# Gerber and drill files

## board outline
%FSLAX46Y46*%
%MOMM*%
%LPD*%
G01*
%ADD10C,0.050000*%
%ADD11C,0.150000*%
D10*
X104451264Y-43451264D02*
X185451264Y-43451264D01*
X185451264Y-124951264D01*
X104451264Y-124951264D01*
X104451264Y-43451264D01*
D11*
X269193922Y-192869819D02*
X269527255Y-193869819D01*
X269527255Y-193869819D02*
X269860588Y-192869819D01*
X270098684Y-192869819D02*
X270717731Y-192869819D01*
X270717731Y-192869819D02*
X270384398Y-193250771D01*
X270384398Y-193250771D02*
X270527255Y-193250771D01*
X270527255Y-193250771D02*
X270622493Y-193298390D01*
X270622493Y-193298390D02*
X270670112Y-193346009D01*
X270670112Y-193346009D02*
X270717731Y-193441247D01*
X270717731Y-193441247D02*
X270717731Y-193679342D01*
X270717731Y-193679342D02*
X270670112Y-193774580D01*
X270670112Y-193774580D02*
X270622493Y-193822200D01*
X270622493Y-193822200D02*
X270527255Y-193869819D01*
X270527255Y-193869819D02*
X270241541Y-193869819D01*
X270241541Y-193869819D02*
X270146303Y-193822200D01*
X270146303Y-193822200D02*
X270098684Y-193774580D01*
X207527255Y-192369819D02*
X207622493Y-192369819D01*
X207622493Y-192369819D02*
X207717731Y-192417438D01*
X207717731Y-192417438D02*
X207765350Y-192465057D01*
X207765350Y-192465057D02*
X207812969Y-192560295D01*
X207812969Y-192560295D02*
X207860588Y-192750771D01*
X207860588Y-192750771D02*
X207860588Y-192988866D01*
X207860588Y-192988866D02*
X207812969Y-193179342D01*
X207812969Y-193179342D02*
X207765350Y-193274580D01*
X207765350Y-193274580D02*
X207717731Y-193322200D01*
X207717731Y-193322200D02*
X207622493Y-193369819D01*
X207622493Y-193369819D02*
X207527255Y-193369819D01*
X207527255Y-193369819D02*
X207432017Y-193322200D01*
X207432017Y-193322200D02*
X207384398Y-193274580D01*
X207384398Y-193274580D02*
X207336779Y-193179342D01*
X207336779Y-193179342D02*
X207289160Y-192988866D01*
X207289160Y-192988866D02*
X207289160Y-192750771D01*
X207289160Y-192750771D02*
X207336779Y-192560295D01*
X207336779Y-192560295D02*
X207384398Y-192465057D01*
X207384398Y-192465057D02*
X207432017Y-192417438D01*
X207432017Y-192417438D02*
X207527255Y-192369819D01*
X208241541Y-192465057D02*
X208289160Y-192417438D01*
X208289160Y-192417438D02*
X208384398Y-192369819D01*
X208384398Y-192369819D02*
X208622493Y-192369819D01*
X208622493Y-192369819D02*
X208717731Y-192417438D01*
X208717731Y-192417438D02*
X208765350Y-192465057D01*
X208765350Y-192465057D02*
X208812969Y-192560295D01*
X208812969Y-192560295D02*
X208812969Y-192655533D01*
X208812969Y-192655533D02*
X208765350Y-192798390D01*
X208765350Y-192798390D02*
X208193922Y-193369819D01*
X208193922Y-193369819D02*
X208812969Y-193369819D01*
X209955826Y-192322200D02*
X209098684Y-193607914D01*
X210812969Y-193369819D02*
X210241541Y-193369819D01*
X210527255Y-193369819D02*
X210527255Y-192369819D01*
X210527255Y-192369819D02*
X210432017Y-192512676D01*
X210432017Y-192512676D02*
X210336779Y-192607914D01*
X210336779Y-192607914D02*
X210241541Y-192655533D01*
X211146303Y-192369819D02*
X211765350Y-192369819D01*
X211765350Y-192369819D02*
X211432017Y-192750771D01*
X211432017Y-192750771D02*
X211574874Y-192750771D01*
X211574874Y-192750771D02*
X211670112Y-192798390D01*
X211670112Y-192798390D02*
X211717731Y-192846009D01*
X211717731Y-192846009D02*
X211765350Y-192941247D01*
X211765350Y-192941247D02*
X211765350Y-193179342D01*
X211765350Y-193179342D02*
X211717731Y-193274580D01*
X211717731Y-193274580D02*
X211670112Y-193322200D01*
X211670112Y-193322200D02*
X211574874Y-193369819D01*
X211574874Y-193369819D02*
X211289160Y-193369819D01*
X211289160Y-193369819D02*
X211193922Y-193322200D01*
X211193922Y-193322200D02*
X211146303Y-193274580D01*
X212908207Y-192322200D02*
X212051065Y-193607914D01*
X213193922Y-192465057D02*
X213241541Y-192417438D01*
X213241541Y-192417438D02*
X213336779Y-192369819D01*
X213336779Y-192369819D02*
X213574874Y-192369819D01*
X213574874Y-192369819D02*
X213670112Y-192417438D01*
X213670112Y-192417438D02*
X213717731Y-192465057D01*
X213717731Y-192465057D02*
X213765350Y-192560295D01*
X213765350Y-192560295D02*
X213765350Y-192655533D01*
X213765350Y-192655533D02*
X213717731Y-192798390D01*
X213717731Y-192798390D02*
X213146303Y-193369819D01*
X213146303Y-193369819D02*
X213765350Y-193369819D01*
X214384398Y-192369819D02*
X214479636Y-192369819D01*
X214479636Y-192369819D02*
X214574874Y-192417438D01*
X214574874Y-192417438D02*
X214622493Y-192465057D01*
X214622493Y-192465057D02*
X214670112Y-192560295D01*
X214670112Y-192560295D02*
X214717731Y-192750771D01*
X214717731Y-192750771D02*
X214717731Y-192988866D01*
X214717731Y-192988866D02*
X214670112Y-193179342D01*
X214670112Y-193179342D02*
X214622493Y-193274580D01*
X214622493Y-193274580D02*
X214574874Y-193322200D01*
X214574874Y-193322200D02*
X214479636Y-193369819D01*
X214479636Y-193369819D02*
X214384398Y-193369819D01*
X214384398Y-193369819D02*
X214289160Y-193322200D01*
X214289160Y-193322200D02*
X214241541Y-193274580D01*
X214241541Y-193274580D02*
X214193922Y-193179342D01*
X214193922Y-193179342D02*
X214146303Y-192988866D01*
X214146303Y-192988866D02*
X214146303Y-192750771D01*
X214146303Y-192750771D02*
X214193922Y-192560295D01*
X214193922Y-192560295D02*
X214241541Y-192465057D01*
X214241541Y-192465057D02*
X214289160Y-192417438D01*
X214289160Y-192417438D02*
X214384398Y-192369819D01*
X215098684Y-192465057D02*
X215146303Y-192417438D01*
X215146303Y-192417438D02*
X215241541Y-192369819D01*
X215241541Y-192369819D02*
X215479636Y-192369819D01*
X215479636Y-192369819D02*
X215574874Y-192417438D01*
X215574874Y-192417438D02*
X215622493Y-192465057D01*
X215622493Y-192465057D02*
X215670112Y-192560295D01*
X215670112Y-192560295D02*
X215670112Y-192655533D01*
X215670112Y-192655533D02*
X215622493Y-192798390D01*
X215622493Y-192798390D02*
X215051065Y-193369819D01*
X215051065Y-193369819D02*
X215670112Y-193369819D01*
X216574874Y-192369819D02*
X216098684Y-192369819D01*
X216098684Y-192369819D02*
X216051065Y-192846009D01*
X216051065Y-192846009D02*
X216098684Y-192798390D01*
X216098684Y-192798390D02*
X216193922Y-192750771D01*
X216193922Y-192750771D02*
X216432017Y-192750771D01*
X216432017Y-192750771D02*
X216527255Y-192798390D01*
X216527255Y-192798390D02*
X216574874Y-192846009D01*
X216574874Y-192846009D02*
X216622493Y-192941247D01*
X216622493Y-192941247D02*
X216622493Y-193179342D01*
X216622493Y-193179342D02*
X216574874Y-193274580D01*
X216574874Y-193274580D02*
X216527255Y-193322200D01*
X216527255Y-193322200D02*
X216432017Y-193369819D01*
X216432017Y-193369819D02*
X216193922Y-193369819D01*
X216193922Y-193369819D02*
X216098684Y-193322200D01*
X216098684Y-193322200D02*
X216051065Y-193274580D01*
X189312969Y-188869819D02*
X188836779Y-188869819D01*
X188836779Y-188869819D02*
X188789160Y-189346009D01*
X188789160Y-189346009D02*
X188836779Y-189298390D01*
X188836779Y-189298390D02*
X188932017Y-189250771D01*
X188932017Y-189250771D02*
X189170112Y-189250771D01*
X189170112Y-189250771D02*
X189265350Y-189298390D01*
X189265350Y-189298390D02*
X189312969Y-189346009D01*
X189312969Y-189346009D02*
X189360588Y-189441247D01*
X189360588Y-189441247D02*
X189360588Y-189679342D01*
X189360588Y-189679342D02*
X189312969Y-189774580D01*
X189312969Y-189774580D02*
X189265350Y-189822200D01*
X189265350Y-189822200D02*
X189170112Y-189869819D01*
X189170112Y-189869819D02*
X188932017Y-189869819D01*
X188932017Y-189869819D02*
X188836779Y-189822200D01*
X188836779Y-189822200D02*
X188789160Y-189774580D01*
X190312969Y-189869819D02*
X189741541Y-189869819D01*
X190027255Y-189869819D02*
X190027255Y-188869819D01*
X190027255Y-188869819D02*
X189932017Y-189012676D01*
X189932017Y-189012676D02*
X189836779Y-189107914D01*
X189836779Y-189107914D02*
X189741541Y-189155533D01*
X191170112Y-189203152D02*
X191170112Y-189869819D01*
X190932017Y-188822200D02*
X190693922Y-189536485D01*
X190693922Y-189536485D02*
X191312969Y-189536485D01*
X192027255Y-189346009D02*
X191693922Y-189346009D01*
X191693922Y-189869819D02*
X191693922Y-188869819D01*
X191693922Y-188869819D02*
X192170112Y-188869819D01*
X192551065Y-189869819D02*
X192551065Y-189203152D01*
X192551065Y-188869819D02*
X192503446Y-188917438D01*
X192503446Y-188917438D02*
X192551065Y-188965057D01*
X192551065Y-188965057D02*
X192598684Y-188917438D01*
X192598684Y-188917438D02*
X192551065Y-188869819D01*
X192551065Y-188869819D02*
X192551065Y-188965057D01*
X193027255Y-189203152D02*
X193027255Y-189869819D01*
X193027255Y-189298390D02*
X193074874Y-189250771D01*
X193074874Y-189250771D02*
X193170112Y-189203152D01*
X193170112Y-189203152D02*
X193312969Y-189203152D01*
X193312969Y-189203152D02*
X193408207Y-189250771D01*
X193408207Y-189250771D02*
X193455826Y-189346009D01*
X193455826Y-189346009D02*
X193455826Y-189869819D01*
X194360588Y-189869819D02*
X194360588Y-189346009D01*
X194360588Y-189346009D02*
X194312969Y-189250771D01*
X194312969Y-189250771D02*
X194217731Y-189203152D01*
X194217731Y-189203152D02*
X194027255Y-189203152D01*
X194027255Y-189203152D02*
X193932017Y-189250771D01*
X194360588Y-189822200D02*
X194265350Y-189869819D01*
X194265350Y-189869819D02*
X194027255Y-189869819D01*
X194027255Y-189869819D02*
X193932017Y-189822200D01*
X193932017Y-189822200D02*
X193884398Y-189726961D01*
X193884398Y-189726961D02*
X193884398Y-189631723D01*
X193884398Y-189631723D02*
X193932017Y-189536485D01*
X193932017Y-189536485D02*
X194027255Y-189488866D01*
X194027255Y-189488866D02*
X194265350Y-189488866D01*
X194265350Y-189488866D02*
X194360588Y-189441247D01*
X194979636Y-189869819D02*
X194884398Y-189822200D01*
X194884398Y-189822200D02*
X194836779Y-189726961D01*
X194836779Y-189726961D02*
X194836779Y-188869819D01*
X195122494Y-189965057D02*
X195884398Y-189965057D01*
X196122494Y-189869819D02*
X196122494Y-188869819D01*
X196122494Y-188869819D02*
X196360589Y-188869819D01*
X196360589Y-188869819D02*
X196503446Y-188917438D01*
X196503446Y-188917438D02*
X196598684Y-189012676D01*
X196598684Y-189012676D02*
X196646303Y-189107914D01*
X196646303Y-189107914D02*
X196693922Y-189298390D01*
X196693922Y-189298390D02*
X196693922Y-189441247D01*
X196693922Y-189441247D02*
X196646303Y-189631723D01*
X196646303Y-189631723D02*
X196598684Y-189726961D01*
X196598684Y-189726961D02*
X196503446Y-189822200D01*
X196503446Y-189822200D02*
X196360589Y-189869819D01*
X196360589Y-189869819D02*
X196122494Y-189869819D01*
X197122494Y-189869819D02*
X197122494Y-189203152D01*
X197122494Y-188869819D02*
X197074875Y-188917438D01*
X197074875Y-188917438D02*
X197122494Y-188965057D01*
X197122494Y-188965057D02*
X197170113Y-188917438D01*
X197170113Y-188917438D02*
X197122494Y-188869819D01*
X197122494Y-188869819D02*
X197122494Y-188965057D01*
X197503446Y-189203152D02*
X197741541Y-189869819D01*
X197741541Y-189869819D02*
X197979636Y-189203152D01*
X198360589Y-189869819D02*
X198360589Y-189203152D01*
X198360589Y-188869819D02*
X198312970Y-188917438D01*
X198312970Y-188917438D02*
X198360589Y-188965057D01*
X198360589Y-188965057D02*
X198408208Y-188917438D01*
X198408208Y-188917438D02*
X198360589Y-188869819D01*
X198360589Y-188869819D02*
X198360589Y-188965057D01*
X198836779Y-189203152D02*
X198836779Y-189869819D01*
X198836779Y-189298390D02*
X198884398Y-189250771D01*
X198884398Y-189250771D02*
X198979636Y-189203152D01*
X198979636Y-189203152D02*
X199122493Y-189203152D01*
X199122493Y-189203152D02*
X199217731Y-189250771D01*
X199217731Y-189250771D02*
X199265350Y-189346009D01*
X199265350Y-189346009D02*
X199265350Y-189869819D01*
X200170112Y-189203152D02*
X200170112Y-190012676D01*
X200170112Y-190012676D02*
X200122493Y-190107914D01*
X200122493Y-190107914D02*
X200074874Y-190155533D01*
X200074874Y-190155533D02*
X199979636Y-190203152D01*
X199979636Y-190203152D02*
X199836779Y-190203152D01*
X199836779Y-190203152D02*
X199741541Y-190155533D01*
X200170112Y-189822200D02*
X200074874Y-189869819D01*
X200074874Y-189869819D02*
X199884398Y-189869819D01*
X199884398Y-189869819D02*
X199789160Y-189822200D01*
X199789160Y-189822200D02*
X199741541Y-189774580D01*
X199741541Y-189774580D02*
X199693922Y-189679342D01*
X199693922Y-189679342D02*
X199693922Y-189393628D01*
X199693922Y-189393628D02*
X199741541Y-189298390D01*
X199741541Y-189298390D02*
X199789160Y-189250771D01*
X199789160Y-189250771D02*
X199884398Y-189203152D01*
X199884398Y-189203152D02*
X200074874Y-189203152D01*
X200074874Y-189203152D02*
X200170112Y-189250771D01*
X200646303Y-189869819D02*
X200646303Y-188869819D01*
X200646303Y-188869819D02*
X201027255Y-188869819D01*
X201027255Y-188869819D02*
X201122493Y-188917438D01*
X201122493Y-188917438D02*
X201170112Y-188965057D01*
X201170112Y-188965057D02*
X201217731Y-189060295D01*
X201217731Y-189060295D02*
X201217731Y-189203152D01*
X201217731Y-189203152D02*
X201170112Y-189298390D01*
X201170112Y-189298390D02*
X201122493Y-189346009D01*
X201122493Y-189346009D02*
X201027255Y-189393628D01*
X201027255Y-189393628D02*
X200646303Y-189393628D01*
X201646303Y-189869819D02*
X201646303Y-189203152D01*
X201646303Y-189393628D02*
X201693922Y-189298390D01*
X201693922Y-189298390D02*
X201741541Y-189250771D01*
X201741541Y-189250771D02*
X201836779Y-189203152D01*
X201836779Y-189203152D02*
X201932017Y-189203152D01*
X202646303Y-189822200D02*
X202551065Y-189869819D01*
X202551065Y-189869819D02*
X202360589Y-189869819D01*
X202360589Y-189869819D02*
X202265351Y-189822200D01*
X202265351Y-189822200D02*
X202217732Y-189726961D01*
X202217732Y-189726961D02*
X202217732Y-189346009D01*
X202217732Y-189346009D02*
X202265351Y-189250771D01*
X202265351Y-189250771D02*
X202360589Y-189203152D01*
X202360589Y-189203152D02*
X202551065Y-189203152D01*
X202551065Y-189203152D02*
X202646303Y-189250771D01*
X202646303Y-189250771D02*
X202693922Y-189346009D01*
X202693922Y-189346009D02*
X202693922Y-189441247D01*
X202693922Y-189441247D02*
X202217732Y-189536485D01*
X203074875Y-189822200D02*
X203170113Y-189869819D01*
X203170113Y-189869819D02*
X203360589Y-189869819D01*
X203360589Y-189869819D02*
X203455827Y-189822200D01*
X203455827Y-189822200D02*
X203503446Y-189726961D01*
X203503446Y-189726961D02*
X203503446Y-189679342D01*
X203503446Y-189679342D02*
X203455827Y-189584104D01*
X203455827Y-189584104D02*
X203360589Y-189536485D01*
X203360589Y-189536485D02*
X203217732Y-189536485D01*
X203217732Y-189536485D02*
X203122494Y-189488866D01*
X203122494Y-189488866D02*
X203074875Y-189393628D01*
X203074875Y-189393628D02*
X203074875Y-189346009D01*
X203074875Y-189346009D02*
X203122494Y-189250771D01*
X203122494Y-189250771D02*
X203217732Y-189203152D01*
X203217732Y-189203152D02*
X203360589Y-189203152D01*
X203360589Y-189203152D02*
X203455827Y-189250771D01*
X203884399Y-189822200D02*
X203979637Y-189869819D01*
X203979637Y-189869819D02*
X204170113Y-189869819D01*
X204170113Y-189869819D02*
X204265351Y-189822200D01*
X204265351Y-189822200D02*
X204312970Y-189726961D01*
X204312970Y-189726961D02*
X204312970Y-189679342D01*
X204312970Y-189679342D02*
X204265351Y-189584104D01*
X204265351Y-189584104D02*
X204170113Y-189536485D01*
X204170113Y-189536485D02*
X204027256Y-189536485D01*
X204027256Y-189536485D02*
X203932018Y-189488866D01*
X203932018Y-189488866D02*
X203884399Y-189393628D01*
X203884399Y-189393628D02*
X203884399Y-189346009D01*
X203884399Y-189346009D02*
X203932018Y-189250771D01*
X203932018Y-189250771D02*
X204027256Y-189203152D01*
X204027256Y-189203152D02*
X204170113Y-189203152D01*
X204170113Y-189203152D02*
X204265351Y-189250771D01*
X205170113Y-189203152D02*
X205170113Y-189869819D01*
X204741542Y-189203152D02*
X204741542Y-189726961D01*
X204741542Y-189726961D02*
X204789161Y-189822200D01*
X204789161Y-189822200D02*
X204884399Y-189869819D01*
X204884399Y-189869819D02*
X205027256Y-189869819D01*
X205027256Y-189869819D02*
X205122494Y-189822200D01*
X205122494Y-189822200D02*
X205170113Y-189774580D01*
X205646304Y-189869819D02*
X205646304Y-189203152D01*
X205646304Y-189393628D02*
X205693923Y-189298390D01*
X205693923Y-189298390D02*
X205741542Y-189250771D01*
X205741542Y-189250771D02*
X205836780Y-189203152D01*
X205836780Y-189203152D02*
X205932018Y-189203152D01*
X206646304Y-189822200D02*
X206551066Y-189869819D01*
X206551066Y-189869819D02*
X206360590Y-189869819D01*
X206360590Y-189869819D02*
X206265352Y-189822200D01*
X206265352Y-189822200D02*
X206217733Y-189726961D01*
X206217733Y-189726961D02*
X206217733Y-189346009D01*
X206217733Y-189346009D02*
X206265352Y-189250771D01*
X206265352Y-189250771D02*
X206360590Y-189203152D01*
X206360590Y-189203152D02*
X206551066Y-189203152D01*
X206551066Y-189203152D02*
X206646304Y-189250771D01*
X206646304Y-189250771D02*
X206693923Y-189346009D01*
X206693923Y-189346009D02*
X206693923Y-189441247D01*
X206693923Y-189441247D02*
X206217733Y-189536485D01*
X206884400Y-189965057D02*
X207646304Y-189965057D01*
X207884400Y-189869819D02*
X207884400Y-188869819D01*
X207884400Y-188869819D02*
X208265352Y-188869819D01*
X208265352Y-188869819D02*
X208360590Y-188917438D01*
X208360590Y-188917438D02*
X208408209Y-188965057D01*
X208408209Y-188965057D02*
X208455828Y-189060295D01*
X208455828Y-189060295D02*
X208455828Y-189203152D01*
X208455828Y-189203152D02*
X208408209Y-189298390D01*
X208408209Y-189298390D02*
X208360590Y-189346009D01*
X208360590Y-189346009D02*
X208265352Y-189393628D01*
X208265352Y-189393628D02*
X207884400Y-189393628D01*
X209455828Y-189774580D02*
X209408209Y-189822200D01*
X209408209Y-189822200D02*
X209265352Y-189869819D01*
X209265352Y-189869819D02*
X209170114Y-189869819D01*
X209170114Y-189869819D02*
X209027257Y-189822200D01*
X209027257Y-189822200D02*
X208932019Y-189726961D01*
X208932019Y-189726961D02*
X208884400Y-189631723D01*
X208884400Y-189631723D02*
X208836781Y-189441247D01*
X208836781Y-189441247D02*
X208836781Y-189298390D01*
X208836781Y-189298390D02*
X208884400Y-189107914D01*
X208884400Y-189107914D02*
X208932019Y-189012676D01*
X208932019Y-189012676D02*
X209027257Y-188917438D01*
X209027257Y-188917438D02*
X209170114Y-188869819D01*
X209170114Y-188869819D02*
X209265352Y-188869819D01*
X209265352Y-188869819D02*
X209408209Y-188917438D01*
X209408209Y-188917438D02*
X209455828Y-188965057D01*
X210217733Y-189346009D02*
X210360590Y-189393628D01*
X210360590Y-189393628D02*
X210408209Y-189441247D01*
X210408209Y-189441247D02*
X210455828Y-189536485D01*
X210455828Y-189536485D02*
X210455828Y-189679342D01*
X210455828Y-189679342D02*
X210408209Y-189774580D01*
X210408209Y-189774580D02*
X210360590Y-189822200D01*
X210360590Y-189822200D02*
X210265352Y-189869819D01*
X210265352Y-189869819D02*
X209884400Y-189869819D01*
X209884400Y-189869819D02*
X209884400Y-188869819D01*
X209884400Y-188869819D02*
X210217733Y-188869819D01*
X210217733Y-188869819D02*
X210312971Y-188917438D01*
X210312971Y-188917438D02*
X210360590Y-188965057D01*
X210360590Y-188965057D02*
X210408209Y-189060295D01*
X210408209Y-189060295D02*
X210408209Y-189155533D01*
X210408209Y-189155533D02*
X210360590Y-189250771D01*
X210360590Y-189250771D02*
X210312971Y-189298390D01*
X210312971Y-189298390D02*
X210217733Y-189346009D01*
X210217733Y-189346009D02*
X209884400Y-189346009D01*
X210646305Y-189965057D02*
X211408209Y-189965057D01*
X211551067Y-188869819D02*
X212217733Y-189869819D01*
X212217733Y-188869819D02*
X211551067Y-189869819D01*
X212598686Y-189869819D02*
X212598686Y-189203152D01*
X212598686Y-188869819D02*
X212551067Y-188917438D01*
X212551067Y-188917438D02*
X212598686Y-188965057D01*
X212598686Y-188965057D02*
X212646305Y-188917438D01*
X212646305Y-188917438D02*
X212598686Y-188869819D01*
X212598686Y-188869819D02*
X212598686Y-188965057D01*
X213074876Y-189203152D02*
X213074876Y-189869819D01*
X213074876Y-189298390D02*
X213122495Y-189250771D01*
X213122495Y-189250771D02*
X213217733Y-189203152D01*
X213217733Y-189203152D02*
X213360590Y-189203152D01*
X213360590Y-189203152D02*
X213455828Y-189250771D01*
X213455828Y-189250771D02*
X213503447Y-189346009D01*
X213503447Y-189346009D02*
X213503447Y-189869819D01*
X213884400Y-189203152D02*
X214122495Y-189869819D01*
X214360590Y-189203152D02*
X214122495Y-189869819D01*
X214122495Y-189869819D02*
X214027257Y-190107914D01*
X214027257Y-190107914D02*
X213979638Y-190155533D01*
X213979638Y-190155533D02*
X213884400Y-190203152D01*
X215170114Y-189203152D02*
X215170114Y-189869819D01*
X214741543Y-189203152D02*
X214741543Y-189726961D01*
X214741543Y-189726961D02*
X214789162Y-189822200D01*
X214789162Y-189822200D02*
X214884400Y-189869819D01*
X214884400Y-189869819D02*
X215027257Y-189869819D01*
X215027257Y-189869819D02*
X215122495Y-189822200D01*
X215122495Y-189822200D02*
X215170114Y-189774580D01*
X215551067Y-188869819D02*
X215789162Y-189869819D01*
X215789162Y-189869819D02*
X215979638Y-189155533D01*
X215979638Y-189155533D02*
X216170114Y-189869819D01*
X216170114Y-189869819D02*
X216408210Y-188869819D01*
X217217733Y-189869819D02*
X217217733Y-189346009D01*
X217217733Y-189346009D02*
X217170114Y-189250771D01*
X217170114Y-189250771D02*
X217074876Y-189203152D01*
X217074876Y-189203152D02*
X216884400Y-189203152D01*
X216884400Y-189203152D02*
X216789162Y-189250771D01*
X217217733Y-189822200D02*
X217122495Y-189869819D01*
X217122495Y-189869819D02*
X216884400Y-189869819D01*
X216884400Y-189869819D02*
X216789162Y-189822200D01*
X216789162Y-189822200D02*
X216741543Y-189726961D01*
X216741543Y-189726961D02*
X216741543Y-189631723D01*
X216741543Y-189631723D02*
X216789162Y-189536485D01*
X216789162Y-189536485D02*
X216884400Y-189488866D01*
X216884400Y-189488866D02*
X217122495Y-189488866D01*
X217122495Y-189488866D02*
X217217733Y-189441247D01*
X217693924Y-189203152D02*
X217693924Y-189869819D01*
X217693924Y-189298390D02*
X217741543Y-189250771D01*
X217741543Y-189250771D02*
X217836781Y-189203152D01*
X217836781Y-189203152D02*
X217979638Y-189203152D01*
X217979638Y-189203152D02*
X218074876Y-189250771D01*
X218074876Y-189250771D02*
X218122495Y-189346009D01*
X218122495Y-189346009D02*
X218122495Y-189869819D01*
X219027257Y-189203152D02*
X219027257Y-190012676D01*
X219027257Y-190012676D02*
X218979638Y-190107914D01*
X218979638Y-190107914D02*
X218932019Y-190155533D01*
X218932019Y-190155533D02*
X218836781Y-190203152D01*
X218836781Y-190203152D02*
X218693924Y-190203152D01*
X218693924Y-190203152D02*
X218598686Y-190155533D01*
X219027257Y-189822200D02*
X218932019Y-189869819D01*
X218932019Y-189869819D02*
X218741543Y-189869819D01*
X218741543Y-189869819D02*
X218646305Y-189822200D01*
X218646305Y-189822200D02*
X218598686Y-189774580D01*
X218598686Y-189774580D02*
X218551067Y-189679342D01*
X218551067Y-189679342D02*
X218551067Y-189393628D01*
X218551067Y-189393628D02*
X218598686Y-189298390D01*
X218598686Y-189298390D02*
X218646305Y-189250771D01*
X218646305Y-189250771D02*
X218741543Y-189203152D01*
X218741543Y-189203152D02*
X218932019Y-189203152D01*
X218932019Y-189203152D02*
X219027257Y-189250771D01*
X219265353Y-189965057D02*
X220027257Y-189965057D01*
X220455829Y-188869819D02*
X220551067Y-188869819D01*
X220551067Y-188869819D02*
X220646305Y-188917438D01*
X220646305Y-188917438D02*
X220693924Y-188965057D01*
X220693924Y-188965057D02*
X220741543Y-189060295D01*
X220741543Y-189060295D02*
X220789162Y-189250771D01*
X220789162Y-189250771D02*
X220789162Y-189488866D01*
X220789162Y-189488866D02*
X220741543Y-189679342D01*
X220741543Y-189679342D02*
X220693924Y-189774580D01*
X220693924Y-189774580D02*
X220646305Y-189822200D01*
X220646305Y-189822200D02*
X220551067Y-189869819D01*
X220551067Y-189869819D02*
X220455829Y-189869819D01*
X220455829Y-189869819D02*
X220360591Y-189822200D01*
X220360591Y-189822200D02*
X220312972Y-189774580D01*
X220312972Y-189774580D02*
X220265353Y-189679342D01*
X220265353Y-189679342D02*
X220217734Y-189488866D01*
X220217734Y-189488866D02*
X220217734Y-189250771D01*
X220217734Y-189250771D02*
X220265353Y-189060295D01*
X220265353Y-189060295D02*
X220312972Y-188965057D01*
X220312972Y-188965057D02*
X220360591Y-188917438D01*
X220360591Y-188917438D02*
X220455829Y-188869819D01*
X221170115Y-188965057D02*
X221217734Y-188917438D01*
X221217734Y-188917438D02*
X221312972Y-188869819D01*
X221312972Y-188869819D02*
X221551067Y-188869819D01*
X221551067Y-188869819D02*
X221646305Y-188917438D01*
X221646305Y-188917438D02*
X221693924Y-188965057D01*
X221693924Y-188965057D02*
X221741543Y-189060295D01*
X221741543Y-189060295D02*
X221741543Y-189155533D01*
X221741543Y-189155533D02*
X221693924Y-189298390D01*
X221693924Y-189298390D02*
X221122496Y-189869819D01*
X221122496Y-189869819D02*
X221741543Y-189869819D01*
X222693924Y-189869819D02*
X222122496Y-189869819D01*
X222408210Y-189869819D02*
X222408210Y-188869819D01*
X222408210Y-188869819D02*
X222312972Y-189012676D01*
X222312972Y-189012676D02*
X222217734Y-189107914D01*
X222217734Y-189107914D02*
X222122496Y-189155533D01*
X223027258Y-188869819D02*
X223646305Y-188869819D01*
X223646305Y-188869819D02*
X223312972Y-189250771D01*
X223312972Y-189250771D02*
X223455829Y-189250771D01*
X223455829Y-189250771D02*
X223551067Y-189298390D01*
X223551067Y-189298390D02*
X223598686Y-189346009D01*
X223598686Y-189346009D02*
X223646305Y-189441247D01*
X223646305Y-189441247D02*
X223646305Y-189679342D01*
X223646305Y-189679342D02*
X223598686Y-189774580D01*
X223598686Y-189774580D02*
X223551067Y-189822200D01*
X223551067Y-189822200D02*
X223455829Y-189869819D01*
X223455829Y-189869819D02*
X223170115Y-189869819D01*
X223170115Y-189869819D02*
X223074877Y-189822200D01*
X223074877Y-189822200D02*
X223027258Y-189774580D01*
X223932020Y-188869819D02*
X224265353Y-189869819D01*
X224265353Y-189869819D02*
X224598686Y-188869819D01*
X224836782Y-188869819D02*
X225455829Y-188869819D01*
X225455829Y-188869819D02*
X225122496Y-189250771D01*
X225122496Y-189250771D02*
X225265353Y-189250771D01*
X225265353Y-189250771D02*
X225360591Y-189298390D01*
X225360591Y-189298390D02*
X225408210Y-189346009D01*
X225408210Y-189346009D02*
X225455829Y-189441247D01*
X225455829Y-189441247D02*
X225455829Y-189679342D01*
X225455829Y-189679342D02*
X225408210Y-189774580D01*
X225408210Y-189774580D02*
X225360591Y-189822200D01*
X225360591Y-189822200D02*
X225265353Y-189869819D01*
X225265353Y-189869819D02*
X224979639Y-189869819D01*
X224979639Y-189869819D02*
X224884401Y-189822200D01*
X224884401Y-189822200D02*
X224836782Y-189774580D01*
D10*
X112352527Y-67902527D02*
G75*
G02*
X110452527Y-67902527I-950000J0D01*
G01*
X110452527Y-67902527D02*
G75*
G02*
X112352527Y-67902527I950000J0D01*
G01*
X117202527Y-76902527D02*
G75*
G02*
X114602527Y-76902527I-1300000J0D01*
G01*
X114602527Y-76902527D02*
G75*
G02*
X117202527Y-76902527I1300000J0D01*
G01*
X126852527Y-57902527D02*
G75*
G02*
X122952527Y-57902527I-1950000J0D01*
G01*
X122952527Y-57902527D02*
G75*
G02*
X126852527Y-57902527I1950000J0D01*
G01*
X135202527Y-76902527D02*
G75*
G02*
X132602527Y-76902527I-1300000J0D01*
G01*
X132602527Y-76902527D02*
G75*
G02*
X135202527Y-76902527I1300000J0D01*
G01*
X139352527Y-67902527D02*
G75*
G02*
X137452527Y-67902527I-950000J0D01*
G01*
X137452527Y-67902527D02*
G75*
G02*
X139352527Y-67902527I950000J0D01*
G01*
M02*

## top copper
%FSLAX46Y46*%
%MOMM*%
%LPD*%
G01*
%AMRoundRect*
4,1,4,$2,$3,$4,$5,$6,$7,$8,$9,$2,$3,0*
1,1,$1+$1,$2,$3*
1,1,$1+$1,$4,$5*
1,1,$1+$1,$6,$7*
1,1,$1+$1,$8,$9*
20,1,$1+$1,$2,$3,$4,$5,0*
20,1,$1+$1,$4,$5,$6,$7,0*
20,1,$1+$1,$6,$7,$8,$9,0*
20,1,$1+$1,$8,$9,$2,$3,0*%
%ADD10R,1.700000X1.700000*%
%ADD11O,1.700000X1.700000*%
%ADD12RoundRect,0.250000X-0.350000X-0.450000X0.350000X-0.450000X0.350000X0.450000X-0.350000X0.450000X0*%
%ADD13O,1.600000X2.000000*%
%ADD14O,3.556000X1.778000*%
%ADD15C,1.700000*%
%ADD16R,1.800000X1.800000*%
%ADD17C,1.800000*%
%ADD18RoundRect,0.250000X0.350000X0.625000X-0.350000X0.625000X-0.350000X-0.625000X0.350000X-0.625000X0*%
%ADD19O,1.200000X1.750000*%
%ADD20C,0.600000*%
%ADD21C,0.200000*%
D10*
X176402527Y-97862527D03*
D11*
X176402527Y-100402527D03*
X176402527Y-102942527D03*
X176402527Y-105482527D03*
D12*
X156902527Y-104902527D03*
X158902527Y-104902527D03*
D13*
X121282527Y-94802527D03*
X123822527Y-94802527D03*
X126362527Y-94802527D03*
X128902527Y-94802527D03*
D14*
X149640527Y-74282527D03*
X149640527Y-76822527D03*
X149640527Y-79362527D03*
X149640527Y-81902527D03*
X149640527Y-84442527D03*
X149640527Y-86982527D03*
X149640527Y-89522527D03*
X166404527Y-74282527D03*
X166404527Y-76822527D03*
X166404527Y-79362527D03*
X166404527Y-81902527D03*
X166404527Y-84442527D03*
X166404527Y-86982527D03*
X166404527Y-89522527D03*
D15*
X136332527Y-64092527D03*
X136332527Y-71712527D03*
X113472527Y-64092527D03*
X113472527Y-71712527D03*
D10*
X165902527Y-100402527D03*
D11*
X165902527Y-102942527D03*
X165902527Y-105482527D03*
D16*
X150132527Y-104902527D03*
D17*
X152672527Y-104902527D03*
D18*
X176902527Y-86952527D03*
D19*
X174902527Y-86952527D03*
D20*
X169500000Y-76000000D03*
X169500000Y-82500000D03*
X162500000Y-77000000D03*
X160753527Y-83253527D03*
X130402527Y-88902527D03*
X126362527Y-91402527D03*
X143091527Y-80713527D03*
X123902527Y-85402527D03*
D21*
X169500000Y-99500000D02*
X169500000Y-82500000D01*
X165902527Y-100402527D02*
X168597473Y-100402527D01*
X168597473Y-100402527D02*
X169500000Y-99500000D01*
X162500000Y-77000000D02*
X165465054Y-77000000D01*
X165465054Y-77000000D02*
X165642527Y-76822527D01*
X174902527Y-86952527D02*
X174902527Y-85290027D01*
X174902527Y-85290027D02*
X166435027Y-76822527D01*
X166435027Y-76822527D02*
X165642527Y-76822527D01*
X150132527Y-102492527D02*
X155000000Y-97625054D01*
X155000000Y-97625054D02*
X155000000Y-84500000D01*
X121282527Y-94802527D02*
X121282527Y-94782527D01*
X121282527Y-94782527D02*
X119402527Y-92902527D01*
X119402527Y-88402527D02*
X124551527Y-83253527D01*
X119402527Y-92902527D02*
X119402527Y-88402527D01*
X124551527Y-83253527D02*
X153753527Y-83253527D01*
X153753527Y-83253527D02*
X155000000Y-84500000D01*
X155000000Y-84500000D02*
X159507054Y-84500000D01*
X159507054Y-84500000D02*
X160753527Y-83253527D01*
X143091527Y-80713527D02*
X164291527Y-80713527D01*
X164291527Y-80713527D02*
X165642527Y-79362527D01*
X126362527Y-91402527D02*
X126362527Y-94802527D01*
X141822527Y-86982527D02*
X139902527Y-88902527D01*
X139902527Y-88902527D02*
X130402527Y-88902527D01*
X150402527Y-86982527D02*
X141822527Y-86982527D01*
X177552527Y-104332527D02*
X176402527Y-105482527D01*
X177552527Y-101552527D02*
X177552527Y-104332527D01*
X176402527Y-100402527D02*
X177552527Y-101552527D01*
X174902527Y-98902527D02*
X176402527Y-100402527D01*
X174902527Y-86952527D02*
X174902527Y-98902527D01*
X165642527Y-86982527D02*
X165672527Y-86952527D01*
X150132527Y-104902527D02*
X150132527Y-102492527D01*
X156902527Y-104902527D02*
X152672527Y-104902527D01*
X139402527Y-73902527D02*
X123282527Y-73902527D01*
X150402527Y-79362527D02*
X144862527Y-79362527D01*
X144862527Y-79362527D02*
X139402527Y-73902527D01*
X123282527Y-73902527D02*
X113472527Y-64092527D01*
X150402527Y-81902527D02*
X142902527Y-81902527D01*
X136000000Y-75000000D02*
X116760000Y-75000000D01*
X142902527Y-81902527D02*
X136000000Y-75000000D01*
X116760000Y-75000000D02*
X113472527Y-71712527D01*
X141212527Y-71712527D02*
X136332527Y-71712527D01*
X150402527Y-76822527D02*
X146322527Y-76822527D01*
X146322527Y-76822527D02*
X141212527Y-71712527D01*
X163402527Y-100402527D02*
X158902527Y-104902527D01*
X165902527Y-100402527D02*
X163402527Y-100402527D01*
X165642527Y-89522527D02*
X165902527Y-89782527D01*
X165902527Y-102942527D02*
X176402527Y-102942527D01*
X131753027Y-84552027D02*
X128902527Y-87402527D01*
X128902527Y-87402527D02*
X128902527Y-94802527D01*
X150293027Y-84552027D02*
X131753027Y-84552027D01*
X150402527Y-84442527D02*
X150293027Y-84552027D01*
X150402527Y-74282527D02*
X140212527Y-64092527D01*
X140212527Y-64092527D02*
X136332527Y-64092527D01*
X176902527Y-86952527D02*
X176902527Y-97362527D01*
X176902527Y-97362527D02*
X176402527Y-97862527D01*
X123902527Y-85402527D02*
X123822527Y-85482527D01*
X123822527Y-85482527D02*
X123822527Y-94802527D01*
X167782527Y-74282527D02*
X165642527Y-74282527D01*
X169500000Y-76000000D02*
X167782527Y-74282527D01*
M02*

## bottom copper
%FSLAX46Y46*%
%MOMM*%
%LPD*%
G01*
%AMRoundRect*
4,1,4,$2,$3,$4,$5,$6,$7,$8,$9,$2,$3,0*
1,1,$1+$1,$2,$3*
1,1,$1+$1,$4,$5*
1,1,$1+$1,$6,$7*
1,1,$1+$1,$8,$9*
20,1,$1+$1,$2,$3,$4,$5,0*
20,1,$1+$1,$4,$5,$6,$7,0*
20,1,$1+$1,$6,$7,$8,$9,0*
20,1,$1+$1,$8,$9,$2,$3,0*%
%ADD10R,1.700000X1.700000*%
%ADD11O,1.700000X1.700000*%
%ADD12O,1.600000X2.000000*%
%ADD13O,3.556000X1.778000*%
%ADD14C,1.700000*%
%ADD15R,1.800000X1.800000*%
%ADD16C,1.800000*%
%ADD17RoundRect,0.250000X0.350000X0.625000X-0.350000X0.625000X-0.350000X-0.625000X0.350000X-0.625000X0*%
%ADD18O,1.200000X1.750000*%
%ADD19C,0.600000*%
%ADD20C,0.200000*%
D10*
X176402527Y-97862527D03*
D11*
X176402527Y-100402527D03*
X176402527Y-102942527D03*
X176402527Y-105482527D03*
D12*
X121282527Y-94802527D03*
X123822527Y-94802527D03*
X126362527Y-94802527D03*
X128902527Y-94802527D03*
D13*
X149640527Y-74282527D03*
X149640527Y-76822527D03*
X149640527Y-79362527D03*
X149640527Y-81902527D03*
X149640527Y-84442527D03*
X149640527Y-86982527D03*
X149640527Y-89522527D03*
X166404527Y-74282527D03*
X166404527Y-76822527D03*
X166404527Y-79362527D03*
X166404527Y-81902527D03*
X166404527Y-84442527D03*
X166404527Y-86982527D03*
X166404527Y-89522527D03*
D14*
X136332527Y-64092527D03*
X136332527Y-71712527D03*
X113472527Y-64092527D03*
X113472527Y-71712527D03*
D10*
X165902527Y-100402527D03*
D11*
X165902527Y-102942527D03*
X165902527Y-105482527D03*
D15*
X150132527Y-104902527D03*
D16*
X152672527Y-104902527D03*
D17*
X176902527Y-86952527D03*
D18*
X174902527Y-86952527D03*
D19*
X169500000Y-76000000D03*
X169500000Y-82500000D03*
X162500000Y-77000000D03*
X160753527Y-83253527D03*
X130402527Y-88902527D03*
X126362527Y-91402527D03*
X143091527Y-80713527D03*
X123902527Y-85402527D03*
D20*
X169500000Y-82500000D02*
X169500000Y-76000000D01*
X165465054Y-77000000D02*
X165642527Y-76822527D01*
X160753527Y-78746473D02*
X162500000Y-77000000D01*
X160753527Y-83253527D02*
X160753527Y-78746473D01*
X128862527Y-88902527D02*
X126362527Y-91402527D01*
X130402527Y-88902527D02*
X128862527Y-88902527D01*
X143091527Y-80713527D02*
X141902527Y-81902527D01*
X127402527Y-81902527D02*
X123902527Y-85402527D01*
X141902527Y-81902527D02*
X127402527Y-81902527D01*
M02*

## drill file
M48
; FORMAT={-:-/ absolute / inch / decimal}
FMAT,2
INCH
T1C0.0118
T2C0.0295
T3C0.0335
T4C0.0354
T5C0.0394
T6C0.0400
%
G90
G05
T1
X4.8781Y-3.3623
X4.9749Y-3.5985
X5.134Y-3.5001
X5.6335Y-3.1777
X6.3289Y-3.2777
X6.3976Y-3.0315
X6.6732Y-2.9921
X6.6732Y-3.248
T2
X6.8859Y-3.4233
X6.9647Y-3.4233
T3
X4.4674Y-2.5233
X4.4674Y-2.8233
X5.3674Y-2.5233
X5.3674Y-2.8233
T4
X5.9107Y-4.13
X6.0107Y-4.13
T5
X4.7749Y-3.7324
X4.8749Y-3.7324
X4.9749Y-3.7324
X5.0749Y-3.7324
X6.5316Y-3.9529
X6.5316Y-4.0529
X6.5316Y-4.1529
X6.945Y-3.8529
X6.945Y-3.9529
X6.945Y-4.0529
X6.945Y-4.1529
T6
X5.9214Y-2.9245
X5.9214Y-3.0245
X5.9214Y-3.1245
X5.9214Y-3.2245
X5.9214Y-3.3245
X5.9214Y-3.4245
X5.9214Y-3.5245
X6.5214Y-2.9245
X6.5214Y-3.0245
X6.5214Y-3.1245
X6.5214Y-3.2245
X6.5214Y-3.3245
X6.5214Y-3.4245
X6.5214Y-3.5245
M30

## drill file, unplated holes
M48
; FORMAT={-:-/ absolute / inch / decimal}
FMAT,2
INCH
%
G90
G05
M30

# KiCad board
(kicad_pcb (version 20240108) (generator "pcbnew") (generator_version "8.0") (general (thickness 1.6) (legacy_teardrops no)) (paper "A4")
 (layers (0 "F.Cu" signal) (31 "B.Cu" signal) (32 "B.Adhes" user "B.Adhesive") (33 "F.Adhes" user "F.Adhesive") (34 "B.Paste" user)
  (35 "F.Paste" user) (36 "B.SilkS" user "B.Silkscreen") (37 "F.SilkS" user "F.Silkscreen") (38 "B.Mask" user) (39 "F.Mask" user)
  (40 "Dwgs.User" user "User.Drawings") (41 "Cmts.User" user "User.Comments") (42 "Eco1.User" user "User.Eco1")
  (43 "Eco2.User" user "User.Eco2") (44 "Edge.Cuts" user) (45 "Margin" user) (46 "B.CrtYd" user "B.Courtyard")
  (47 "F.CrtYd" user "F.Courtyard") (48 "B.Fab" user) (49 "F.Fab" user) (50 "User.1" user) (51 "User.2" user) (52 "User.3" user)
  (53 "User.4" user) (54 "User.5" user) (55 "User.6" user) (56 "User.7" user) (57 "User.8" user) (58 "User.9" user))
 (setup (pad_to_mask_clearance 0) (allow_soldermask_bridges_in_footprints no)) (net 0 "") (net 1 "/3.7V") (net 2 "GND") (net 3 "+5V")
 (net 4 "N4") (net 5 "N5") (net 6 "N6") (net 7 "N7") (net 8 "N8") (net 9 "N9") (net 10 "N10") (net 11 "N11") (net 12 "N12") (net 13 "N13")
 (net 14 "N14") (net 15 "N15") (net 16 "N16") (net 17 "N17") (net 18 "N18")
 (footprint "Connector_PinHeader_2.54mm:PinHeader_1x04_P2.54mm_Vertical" (layer "F.Cu") (at 176.402527 97.862527)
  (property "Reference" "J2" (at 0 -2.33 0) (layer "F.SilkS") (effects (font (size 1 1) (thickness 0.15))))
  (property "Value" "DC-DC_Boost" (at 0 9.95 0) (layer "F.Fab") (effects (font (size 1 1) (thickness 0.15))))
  (pad "1" thru_hole rect (at 0 0) (size 1.7 1.7) (drill 1) (layers "*.Cu" "*.Mask") (remove_unused_layers no) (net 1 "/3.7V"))
  (pad "2" thru_hole oval (at 0 2.54) (size 1.7 1.7) (drill 1) (layers "*.Cu" "*.Mask") (remove_unused_layers no) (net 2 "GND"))
  (pad "3" thru_hole oval (at 0 5.08) (size 1.7 1.7) (drill 1) (layers "*.Cu" "*.Mask") (remove_unused_layers no) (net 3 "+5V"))
  (pad "4" thru_hole oval (at 0 7.62) (size 1.7 1.7) (drill 1) (layers "*.Cu" "*.Mask") (remove_unused_layers no) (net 2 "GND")))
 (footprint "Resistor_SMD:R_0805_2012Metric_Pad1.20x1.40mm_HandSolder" (layer "F.Cu") (at 157.902527 104.902527)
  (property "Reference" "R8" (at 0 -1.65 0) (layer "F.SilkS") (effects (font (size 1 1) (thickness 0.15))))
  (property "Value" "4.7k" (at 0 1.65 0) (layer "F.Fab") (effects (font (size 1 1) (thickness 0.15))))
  (pad "1" smd roundrect (at -1 0) (size 1.2 1.4) (layers "F.Cu" "F.Paste" "F.Mask") (roundrect_rratio 0.208333) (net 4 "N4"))
  (pad "2" smd roundrect (at 1 0) (size 1.2 1.4) (layers "F.Cu" "F.Paste" "F.Mask") (roundrect_rratio 0.208333) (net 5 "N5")))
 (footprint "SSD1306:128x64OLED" (layer "F.Cu") (at 124.902527 105.402527)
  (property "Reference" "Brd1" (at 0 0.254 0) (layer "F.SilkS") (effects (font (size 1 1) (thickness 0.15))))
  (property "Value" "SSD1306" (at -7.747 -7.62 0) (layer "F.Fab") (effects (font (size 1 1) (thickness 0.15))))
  (pad "1" thru_hole oval (at -3.62 -10.6 90) (size 2 1.6) (drill 1) (layers "*.Cu" "*.Mask") (remove_unused_layers no) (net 2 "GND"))
  (pad "2" thru_hole oval (at -1.08 -10.6 90) (size 2 1.6) (drill 1) (layers "*.Cu" "*.Mask") (remove_unused_layers no) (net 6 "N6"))
  (pad "3" thru_hole oval (at 1.46 -10.6 90) (size 2 1.6) (drill 1) (layers "*.Cu" "*.Mask") (remove_unused_layers no) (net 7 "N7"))
  (pad "4" thru_hole oval (at 4 -10.6 90) (size 2 1.6) (drill 1) (layers "*.Cu" "*.Mask") (remove_unused_layers no) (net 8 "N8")))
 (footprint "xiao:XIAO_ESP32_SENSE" (layer "F.Cu") (at 158.022527 81.902527)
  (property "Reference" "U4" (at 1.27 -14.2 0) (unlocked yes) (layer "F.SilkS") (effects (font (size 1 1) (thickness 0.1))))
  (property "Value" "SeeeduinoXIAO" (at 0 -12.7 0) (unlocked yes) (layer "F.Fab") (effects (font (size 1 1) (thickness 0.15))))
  (pad "1" thru_hole oval (at -7.62 -7.62) (size 3.556 1.778) (drill 1.016 (offset -0.762 0)) (layers "*.Cu" "*.Mask")
   (remove_unused_layers no) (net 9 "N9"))
  (pad "2" thru_hole oval (at -7.62 -5.08) (size 3.556 1.778) (drill 1.016 (offset -0.762 0)) (layers "*.Cu" "*.Mask")
   (remove_unused_layers no) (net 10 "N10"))
  (pad "3" thru_hole oval (at -7.62 -2.54) (size 3.556 1.778) (drill 1.016 (offset -0.762 0)) (layers "*.Cu" "*.Mask")
   (remove_unused_layers no) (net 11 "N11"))
  (pad "4" thru_hole oval (at -7.62 0) (size 3.556 1.778) (drill 1.016 (offset -0.762 0)) (layers "*.Cu" "*.Mask") (remove_unused_layers no)
   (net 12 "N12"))
  (pad "5" thru_hole oval (at -7.62 2.54) (size 3.556 1.778) (drill 1.016 (offset -0.762 0)) (layers "*.Cu" "*.Mask")
   (remove_unused_layers no) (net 8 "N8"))
  (pad "6" thru_hole oval (at -7.62 5.08) (size 3.556 1.778) (drill 1.016 (offset -0.762 0)) (layers "*.Cu" "*.Mask")
   (remove_unused_layers no) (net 7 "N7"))
  (pad "7" thru_hole oval (at -7.62 7.62) (size 3.556 1.778) (drill 1.016 (offset -0.762 0)) (layers "*.Cu" "*.Mask")
   (remove_unused_layers no) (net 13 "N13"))
  (pad "8" thru_hole oval (at 7.62 -7.62) (size 3.556 1.778) (drill 1.016 (offset 0.762 0)) (layers "*.Cu" "*.Mask")
   (remove_unused_layers no) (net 5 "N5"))
  (pad "9" thru_hole oval (at 7.62 -5.08) (size 3.556 1.778) (drill 1.016 (offset 0.762 0)) (layers "*.Cu" "*.Mask")
   (remove_unused_layers no) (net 2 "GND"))
  (pad "10" thru_hole oval (at 7.62 -2.54) (size 3.556 1.778) (drill 1.016 (offset 0.762 0)) (layers "*.Cu" "*.Mask")
   (remove_unused_layers no) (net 6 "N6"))
  (pad "11" thru_hole oval (at 7.62 0) (size 3.556 1.778) (drill 1.016 (offset 0.762 0)) (layers "*.Cu" "*.Mask") (remove_unused_layers no)
   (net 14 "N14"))
  (pad "12" thru_hole oval (at 7.62 2.54) (size 3.556 1.778) (drill 1.016 (offset 0.762 0)) (layers "*.Cu" "*.Mask")
   (remove_unused_layers no) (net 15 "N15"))
  (pad "13" thru_hole oval (at 7.62 5.08) (size 3.556 1.778) (drill 1.016 (offset 0.762 0)) (layers "*.Cu" "*.Mask")
   (remove_unused_layers no) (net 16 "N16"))
  (pad "14" thru_hole oval (at 7.62 7.62) (size 3.556 1.778) (drill 1.016 (offset 0.762 0)) (layers "*.Cu" "*.Mask")
   (remove_unused_layers no) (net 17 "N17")))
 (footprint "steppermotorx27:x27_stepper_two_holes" (layer "F.Cu") (at 127.442527 78.062527)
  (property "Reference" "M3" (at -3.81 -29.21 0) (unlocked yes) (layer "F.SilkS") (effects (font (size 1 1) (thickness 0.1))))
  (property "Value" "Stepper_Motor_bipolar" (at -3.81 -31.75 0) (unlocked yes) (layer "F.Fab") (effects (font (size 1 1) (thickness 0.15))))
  (fp_circle (center -16.04 -10.16) (end -15.09 -10.16) (stroke (width 0.05) (type default)) (fill none) (layer "Edge.Cuts"))
  (fp_circle (center -11.54 -1.16) (end -10.24 -1.16) (stroke (width 0.05) (type default)) (fill none) (layer "Edge.Cuts"))
  (fp_circle (center -2.54 -20.16) (end -0.59 -20.16) (stroke (width 0.05) (type default)) (fill none) (layer "Edge.Cuts"))
  (fp_circle (center 6.46 -1.16) (end 7.76 -1.16) (stroke (width 0.05) (type default)) (fill none) (layer "Edge.Cuts"))
  (fp_circle (center 10.96 -10.16) (end 11.91 -10.16) (stroke (width 0.05) (type default)) (fill none) (layer "Edge.Cuts"))
  (pad "1" thru_hole circle (at 8.89 -13.97) (size 1.7 1.7) (drill 0.85) (layers "*.Cu" "*.Mask") (remove_unused_layers no) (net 9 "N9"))
  (pad "2" thru_hole circle (at 8.89 -6.35) (size 1.7 1.7) (drill 0.85) (layers "*.Cu" "*.Mask") (remove_unused_layers no) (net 10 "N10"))
  (pad "3" thru_hole circle (at -13.97 -13.97) (size 1.7 1.7) (drill 0.85) (layers "*.Cu" "*.Mask") (remove_unused_layers no) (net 11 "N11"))
  (pad "4" thru_hole circle (at -13.97 -6.35) (size 1.7 1.7) (drill 0.85) (layers "*.Cu" "*.Mask") (remove_unused_layers no) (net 12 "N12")))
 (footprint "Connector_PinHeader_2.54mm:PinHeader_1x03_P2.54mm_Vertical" (layer "F.Cu") (at 165.902527 100.402527)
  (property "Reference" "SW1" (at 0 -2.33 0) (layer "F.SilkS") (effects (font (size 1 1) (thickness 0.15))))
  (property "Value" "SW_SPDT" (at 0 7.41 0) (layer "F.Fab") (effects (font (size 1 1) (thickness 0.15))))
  (pad "1" thru_hole rect (at 0 0) (size 1.7 1.7) (drill 1) (layers "*.Cu" "*.Mask") (remove_unused_layers no) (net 5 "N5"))
  (pad "2" thru_hole oval (at 0 2.54) (size 1.7 1.7) (drill 1) (layers "*.Cu" "*.Mask") (remove_unused_layers no) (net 3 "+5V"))
  (pad "3" thru_hole oval (at 0 5.08) (size 1.7 1.7) (drill 1) (layers "*.Cu" "*.Mask") (remove_unused_layers no) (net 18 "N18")))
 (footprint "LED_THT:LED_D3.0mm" (layer "F.Cu") (at 150.132527 104.902527)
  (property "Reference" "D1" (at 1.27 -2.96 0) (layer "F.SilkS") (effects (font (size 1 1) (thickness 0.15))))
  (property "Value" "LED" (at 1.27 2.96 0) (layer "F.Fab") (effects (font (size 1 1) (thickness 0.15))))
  (pad "1" thru_hole rect (at 0 0) (size 1.8 1.8) (drill 0.9) (layers "*.Cu" "*.Mask") (remove_unused_layers no) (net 2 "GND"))
  (pad "2" thru_hole circle (at 2.54 0) (size 1.8 1.8) (drill 0.9) (layers "*.Cu" "*.Mask") (remove_unused_layers no) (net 4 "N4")))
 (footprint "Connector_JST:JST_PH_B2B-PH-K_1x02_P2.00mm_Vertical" (layer "F.Cu") (at 176.902527 86.952527 180)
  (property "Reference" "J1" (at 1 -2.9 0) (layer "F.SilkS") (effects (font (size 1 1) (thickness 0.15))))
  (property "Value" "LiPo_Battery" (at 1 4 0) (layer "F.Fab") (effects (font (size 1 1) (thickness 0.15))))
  (pad "1" thru_hole roundrect (at 0 0 180) (size 1.2 1.75) (drill 0.75) (layers "*.Cu" "*.Mask") (remove_unused_layers no)
   (roundrect_rratio 0.208333) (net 1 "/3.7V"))
  (pad "2" thru_hole oval (at 2 0 180) (size 1.2 1.75) (drill 0.75) (layers "*.Cu" "*.Mask") (remove_unused_layers no) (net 2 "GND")))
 (gr_rect (start 104.451264 43.451264) (end 185.451264 124.951264) (stroke (width 0.05) (type default)) (fill none) (layer "Edge.Cuts"))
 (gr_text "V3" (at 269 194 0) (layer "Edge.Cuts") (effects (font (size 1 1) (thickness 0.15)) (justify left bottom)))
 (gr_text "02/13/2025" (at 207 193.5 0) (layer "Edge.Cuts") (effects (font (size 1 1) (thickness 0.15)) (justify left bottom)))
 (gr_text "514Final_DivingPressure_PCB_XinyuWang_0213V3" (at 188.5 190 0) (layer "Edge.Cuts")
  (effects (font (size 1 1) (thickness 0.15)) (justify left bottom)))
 (segment (start 126.362527 91.402527) (end 126.362527 94.802527) (width 0.2) (layer "F.Cu") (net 7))
 (segment (start 141.822527 86.982527) (end 139.902527 88.902527) (width 0.2) (layer "F.Cu") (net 7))
 (segment (start 139.902527 88.902527) (end 130.402527 88.902527) (width 0.2) (layer "F.Cu") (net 7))
 (segment (start 150.402527 86.982527) (end 141.822527 86.982527) (width 0.2) (layer "F.Cu") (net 7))
 (via (at 130.402527 88.902527) (size 0.6) (drill 0.3) (layers "F.Cu" "B.Cu") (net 7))
 (via (at 126.362527 91.402527) (size 0.6) (drill 0.3) (layers "F.Cu" "B.Cu") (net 7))
 (segment (start 128.862527 88.902527) (end 126.362527 91.402527) (width 0.2) (layer "B.Cu") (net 7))
 (segment (start 130.402527 88.902527) (end 128.862527 88.902527) (width 0.2) (layer "B.Cu") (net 7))
 (segment (start 177.552527 104.332527) (end 176.402527 105.482527) (width 0.2) (layer "F.Cu") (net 2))
 (segment (start 177.552527 101.552527) (end 177.552527 104.332527) (width 0.2) (layer "F.Cu") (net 2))
 (segment (start 150.132527 102.492527) (end 155 97.625054) (width 0.2) (layer "F.Cu") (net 2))
 (segment (start 166.435027 76.822527) (end 165.642527 76.822527) (width 0.2) (layer "F.Cu") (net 2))
 (segment (start 153.753527 83.253527) (end 155 84.5) (width 0.2) (layer "F.Cu") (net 2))
 (segment (start 155 97.625054) (end 155 84.5) (width 0.2) (layer "F.Cu") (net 2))
 (segment (start 159.507054 84.5) (end 160.753527 83.253527) (width 0.2) (layer "F.Cu") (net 2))
 (segment (start 176.402527 100.402527) (end 177.552527 101.552527) (width 0.2) (layer "F.Cu") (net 2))
 (segment (start 174.902527 98.902527) (end 176.402527 100.402527) (width 0.2) (layer "F.Cu") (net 2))
 (segment (start 174.902527 85.290027) (end 166.435027 76.822527) (width 0.2) (layer "F.Cu") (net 2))
 (segment (start 174.902527 86.952527) (end 174.902527 98.902527) (width 0.2) (layer "F.Cu") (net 2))
 (segment (start 119.402527 92.902527) (end 119.402527 88.402527) (width 0.2) (layer "F.Cu") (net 2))
 (segment (start 119.402527 88.402527) (end 124.551527 83.253527) (width 0.2) (layer "F.Cu") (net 2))
 (segment (start 162.5 77) (end 165.465054 77) (width 0.2) (layer "F.Cu") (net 2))
 (segment (start 165.465054 77) (end 165.642527 76.822527) (width 0.2) (layer "F.Cu") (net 2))
 (segment (start 121.282527 94.782527) (end 119.402527 92.902527) (width 0.2) (layer "F.Cu") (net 2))
 (segment (start 121.282527 94.802527) (end 121.282527 94.782527) (width 0.2) (layer "F.Cu") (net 2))
 (segment (start 155 84.5) (end 159.507054 84.5) (width 0.2) (layer "F.Cu") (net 2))
 (segment (start 174.902527 86.952527) (end 174.902527 85.290027) (width 0.2) (layer "F.Cu") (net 2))
 (segment (start 124.551527 83.253527) (end 153.753527 83.253527) (width 0.2) (layer "F.Cu") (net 2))
 (segment (start 150.132527 104.902527) (end 150.132527 102.492527) (width 0.2) (layer "F.Cu") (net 2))
 (via (at 162.5 77) (size 0.6) (drill 0.3) (layers "F.Cu" "B.Cu") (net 2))
 (via (at 160.753527 83.253527) (size 0.6) (drill 0.3) (layers "F.Cu" "B.Cu") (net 2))
 (segment (start 160.753527 78.746473) (end 162.5 77) (width 0.2) (layer "B.Cu") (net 2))
 (segment (start 160.753527 83.253527) (end 160.753527 78.746473) (width 0.2) (layer "B.Cu") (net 2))
 (segment (start 165.465054 77) (end 165.642527 76.822527) (width 0.2) (layer "B.Cu") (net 2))
 (segment (start 156.902527 104.902527) (end 152.672527 104.902527) (width 0.2) (layer "F.Cu") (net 4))
 (segment (start 139.402527 73.902527) (end 123.282527 73.902527) (width 0.2) (layer "F.Cu") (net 11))
 (segment (start 150.402527 79.362527) (end 144.862527 79.362527) (width 0.2) (layer "F.Cu") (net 11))
 (segment (start 144.862527 79.362527) (end 139.402527 73.902527) (width 0.2) (layer "F.Cu") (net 11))
 (segment (start 123.282527 73.902527) (end 113.472527 64.092527) (width 0.2) (layer "F.Cu") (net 11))
 (segment (start 150.402527 81.902527) (end 142.902527 81.902527) (width 0.2) (layer "F.Cu") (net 12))
 (segment (start 136 75) (end 116.76 75) (width 0.2) (layer "F.Cu") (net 12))
 (segment (start 142.902527 81.902527) (end 136 75) (width 0.2) (layer "F.Cu") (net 12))
 (segment (start 116.76 75) (end 113.472527 71.712527) (width 0.2) (layer "F.Cu") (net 12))
 (segment (start 141.212527 71.712527) (end 136.332527 71.712527) (width 0.2) (layer "F.Cu") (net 10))
 (segment (start 150.402527 76.822527) (end 146.322527 76.822527) (width 0.2) (layer "F.Cu") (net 10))
 (segment (start 146.322527 76.822527) (end 141.212527 71.712527) (width 0.2) (layer "F.Cu") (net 10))
 (segment (start 163.402527 100.402527) (end 158.902527 104.902527) (width 0.2) (layer "F.Cu") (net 5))
 (segment (start 165.902527 100.402527) (end 163.402527 100.402527) (width 0.2) (layer "F.Cu") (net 5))
 (segment (start 169.5 99.5) (end 169.5 82.5) (width 0.2) (layer "F.Cu") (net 5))
 (segment (start 169.5 76) (end 167.782527 74.282527) (width 0.2) (layer "F.Cu") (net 5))
 (segment (start 165.902527 100.402527) (end 168.597473 100.402527) (width 0.2) (layer "F.Cu") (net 5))
 (segment (start 167.782527 74.282527) (end 165.642527 74.282527) (width 0.2) (layer "F.Cu") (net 5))
 (segment (start 168.597473 100.402527) (end 169.5 99.5) (width 0.2) (layer "F.Cu") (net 5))
 (via (at 169.5 76) (size 0.6) (drill 0.3) (layers "F.Cu" "B.Cu") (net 5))
 (via (at 169.5 82.5) (size 0.6) (drill 0.3) (layers "F.Cu" "B.Cu") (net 5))
 (segment (start 169.5 82.5) (end 169.5 76) (width 0.2) (layer "B.Cu") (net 5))
 (segment (start 165.902527 102.942527) (end 176.402527 102.942527) (width 0.2) (layer "F.Cu") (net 3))
 (segment (start 131.753027 84.552027) (end 128.902527 87.402527) (width 0.2) (layer "F.Cu") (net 8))
 (segment (start 128.902527 87.402527) (end 128.902527 94.802527) (width 0.2) (layer "F.Cu") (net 8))
 (segment (start 150.293027 84.552027) (end 131.753027 84.552027) (width 0.2) (layer "F.Cu") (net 8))
 (segment (start 150.402527 84.442527) (end 150.293027 84.552027) (width 0.2) (layer "F.Cu") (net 8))
 (segment (start 150.402527 74.282527) (end 140.212527 64.092527) (width 0.2) (layer "F.Cu") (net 9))
 (segment (start 140.212527 64.092527) (end 136.332527 64.092527) (width 0.2) (layer "F.Cu") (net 9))
 (segment (start 165.642527 86.982527) (end 165.672527 86.952527) (width 0.2) (layer "F.Cu") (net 16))
 (segment (start 165.642527 89.522527) (end 165.902527 89.782527) (width 0.2) (layer "F.Cu") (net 17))
 (segment (start 176.902527 86.952527) (end 176.902527 97.362527) (width 0.2) (layer "F.Cu") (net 1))
 (segment (start 176.902527 97.362527) (end 176.402527 97.862527) (width 0.2) (layer "F.Cu") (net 1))
 (segment (start 143.091527 80.713527) (end 164.291527 80.713527) (width 0.2) (layer "F.Cu") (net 6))
 (segment (start 164.291527 80.713527) (end 165.642527 79.362527) (width 0.2) (layer "F.Cu") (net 6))
 (segment (start 123.902527 85.402527) (end 123.822527 85.482527) (width 0.2) (layer "F.Cu") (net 6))
 (segment (start 123.822527 85.482527) (end 123.822527 94.802527) (width 0.2) (layer "F.Cu") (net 6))
 (via (at 143.091527 80.713527) (size 0.6) (drill 0.3) (layers "F.Cu" "B.Cu") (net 6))
 (via (at 123.902527 85.402527) (size 0.6) (drill 0.3) (layers "F.Cu" "B.Cu") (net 6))
 (segment (start 143.091527 80.713527) (end 141.902527 81.902527) (width 0.2) (layer "B.Cu") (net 6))
 (segment (start 127.402527 81.902527) (end 123.902527 85.402527) (width 0.2) (layer "B.Cu") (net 6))
 (segment (start 141.902527 81.902527) (end 127.402527 81.902527) (width 0.2) (layer "B.Cu") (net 6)))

